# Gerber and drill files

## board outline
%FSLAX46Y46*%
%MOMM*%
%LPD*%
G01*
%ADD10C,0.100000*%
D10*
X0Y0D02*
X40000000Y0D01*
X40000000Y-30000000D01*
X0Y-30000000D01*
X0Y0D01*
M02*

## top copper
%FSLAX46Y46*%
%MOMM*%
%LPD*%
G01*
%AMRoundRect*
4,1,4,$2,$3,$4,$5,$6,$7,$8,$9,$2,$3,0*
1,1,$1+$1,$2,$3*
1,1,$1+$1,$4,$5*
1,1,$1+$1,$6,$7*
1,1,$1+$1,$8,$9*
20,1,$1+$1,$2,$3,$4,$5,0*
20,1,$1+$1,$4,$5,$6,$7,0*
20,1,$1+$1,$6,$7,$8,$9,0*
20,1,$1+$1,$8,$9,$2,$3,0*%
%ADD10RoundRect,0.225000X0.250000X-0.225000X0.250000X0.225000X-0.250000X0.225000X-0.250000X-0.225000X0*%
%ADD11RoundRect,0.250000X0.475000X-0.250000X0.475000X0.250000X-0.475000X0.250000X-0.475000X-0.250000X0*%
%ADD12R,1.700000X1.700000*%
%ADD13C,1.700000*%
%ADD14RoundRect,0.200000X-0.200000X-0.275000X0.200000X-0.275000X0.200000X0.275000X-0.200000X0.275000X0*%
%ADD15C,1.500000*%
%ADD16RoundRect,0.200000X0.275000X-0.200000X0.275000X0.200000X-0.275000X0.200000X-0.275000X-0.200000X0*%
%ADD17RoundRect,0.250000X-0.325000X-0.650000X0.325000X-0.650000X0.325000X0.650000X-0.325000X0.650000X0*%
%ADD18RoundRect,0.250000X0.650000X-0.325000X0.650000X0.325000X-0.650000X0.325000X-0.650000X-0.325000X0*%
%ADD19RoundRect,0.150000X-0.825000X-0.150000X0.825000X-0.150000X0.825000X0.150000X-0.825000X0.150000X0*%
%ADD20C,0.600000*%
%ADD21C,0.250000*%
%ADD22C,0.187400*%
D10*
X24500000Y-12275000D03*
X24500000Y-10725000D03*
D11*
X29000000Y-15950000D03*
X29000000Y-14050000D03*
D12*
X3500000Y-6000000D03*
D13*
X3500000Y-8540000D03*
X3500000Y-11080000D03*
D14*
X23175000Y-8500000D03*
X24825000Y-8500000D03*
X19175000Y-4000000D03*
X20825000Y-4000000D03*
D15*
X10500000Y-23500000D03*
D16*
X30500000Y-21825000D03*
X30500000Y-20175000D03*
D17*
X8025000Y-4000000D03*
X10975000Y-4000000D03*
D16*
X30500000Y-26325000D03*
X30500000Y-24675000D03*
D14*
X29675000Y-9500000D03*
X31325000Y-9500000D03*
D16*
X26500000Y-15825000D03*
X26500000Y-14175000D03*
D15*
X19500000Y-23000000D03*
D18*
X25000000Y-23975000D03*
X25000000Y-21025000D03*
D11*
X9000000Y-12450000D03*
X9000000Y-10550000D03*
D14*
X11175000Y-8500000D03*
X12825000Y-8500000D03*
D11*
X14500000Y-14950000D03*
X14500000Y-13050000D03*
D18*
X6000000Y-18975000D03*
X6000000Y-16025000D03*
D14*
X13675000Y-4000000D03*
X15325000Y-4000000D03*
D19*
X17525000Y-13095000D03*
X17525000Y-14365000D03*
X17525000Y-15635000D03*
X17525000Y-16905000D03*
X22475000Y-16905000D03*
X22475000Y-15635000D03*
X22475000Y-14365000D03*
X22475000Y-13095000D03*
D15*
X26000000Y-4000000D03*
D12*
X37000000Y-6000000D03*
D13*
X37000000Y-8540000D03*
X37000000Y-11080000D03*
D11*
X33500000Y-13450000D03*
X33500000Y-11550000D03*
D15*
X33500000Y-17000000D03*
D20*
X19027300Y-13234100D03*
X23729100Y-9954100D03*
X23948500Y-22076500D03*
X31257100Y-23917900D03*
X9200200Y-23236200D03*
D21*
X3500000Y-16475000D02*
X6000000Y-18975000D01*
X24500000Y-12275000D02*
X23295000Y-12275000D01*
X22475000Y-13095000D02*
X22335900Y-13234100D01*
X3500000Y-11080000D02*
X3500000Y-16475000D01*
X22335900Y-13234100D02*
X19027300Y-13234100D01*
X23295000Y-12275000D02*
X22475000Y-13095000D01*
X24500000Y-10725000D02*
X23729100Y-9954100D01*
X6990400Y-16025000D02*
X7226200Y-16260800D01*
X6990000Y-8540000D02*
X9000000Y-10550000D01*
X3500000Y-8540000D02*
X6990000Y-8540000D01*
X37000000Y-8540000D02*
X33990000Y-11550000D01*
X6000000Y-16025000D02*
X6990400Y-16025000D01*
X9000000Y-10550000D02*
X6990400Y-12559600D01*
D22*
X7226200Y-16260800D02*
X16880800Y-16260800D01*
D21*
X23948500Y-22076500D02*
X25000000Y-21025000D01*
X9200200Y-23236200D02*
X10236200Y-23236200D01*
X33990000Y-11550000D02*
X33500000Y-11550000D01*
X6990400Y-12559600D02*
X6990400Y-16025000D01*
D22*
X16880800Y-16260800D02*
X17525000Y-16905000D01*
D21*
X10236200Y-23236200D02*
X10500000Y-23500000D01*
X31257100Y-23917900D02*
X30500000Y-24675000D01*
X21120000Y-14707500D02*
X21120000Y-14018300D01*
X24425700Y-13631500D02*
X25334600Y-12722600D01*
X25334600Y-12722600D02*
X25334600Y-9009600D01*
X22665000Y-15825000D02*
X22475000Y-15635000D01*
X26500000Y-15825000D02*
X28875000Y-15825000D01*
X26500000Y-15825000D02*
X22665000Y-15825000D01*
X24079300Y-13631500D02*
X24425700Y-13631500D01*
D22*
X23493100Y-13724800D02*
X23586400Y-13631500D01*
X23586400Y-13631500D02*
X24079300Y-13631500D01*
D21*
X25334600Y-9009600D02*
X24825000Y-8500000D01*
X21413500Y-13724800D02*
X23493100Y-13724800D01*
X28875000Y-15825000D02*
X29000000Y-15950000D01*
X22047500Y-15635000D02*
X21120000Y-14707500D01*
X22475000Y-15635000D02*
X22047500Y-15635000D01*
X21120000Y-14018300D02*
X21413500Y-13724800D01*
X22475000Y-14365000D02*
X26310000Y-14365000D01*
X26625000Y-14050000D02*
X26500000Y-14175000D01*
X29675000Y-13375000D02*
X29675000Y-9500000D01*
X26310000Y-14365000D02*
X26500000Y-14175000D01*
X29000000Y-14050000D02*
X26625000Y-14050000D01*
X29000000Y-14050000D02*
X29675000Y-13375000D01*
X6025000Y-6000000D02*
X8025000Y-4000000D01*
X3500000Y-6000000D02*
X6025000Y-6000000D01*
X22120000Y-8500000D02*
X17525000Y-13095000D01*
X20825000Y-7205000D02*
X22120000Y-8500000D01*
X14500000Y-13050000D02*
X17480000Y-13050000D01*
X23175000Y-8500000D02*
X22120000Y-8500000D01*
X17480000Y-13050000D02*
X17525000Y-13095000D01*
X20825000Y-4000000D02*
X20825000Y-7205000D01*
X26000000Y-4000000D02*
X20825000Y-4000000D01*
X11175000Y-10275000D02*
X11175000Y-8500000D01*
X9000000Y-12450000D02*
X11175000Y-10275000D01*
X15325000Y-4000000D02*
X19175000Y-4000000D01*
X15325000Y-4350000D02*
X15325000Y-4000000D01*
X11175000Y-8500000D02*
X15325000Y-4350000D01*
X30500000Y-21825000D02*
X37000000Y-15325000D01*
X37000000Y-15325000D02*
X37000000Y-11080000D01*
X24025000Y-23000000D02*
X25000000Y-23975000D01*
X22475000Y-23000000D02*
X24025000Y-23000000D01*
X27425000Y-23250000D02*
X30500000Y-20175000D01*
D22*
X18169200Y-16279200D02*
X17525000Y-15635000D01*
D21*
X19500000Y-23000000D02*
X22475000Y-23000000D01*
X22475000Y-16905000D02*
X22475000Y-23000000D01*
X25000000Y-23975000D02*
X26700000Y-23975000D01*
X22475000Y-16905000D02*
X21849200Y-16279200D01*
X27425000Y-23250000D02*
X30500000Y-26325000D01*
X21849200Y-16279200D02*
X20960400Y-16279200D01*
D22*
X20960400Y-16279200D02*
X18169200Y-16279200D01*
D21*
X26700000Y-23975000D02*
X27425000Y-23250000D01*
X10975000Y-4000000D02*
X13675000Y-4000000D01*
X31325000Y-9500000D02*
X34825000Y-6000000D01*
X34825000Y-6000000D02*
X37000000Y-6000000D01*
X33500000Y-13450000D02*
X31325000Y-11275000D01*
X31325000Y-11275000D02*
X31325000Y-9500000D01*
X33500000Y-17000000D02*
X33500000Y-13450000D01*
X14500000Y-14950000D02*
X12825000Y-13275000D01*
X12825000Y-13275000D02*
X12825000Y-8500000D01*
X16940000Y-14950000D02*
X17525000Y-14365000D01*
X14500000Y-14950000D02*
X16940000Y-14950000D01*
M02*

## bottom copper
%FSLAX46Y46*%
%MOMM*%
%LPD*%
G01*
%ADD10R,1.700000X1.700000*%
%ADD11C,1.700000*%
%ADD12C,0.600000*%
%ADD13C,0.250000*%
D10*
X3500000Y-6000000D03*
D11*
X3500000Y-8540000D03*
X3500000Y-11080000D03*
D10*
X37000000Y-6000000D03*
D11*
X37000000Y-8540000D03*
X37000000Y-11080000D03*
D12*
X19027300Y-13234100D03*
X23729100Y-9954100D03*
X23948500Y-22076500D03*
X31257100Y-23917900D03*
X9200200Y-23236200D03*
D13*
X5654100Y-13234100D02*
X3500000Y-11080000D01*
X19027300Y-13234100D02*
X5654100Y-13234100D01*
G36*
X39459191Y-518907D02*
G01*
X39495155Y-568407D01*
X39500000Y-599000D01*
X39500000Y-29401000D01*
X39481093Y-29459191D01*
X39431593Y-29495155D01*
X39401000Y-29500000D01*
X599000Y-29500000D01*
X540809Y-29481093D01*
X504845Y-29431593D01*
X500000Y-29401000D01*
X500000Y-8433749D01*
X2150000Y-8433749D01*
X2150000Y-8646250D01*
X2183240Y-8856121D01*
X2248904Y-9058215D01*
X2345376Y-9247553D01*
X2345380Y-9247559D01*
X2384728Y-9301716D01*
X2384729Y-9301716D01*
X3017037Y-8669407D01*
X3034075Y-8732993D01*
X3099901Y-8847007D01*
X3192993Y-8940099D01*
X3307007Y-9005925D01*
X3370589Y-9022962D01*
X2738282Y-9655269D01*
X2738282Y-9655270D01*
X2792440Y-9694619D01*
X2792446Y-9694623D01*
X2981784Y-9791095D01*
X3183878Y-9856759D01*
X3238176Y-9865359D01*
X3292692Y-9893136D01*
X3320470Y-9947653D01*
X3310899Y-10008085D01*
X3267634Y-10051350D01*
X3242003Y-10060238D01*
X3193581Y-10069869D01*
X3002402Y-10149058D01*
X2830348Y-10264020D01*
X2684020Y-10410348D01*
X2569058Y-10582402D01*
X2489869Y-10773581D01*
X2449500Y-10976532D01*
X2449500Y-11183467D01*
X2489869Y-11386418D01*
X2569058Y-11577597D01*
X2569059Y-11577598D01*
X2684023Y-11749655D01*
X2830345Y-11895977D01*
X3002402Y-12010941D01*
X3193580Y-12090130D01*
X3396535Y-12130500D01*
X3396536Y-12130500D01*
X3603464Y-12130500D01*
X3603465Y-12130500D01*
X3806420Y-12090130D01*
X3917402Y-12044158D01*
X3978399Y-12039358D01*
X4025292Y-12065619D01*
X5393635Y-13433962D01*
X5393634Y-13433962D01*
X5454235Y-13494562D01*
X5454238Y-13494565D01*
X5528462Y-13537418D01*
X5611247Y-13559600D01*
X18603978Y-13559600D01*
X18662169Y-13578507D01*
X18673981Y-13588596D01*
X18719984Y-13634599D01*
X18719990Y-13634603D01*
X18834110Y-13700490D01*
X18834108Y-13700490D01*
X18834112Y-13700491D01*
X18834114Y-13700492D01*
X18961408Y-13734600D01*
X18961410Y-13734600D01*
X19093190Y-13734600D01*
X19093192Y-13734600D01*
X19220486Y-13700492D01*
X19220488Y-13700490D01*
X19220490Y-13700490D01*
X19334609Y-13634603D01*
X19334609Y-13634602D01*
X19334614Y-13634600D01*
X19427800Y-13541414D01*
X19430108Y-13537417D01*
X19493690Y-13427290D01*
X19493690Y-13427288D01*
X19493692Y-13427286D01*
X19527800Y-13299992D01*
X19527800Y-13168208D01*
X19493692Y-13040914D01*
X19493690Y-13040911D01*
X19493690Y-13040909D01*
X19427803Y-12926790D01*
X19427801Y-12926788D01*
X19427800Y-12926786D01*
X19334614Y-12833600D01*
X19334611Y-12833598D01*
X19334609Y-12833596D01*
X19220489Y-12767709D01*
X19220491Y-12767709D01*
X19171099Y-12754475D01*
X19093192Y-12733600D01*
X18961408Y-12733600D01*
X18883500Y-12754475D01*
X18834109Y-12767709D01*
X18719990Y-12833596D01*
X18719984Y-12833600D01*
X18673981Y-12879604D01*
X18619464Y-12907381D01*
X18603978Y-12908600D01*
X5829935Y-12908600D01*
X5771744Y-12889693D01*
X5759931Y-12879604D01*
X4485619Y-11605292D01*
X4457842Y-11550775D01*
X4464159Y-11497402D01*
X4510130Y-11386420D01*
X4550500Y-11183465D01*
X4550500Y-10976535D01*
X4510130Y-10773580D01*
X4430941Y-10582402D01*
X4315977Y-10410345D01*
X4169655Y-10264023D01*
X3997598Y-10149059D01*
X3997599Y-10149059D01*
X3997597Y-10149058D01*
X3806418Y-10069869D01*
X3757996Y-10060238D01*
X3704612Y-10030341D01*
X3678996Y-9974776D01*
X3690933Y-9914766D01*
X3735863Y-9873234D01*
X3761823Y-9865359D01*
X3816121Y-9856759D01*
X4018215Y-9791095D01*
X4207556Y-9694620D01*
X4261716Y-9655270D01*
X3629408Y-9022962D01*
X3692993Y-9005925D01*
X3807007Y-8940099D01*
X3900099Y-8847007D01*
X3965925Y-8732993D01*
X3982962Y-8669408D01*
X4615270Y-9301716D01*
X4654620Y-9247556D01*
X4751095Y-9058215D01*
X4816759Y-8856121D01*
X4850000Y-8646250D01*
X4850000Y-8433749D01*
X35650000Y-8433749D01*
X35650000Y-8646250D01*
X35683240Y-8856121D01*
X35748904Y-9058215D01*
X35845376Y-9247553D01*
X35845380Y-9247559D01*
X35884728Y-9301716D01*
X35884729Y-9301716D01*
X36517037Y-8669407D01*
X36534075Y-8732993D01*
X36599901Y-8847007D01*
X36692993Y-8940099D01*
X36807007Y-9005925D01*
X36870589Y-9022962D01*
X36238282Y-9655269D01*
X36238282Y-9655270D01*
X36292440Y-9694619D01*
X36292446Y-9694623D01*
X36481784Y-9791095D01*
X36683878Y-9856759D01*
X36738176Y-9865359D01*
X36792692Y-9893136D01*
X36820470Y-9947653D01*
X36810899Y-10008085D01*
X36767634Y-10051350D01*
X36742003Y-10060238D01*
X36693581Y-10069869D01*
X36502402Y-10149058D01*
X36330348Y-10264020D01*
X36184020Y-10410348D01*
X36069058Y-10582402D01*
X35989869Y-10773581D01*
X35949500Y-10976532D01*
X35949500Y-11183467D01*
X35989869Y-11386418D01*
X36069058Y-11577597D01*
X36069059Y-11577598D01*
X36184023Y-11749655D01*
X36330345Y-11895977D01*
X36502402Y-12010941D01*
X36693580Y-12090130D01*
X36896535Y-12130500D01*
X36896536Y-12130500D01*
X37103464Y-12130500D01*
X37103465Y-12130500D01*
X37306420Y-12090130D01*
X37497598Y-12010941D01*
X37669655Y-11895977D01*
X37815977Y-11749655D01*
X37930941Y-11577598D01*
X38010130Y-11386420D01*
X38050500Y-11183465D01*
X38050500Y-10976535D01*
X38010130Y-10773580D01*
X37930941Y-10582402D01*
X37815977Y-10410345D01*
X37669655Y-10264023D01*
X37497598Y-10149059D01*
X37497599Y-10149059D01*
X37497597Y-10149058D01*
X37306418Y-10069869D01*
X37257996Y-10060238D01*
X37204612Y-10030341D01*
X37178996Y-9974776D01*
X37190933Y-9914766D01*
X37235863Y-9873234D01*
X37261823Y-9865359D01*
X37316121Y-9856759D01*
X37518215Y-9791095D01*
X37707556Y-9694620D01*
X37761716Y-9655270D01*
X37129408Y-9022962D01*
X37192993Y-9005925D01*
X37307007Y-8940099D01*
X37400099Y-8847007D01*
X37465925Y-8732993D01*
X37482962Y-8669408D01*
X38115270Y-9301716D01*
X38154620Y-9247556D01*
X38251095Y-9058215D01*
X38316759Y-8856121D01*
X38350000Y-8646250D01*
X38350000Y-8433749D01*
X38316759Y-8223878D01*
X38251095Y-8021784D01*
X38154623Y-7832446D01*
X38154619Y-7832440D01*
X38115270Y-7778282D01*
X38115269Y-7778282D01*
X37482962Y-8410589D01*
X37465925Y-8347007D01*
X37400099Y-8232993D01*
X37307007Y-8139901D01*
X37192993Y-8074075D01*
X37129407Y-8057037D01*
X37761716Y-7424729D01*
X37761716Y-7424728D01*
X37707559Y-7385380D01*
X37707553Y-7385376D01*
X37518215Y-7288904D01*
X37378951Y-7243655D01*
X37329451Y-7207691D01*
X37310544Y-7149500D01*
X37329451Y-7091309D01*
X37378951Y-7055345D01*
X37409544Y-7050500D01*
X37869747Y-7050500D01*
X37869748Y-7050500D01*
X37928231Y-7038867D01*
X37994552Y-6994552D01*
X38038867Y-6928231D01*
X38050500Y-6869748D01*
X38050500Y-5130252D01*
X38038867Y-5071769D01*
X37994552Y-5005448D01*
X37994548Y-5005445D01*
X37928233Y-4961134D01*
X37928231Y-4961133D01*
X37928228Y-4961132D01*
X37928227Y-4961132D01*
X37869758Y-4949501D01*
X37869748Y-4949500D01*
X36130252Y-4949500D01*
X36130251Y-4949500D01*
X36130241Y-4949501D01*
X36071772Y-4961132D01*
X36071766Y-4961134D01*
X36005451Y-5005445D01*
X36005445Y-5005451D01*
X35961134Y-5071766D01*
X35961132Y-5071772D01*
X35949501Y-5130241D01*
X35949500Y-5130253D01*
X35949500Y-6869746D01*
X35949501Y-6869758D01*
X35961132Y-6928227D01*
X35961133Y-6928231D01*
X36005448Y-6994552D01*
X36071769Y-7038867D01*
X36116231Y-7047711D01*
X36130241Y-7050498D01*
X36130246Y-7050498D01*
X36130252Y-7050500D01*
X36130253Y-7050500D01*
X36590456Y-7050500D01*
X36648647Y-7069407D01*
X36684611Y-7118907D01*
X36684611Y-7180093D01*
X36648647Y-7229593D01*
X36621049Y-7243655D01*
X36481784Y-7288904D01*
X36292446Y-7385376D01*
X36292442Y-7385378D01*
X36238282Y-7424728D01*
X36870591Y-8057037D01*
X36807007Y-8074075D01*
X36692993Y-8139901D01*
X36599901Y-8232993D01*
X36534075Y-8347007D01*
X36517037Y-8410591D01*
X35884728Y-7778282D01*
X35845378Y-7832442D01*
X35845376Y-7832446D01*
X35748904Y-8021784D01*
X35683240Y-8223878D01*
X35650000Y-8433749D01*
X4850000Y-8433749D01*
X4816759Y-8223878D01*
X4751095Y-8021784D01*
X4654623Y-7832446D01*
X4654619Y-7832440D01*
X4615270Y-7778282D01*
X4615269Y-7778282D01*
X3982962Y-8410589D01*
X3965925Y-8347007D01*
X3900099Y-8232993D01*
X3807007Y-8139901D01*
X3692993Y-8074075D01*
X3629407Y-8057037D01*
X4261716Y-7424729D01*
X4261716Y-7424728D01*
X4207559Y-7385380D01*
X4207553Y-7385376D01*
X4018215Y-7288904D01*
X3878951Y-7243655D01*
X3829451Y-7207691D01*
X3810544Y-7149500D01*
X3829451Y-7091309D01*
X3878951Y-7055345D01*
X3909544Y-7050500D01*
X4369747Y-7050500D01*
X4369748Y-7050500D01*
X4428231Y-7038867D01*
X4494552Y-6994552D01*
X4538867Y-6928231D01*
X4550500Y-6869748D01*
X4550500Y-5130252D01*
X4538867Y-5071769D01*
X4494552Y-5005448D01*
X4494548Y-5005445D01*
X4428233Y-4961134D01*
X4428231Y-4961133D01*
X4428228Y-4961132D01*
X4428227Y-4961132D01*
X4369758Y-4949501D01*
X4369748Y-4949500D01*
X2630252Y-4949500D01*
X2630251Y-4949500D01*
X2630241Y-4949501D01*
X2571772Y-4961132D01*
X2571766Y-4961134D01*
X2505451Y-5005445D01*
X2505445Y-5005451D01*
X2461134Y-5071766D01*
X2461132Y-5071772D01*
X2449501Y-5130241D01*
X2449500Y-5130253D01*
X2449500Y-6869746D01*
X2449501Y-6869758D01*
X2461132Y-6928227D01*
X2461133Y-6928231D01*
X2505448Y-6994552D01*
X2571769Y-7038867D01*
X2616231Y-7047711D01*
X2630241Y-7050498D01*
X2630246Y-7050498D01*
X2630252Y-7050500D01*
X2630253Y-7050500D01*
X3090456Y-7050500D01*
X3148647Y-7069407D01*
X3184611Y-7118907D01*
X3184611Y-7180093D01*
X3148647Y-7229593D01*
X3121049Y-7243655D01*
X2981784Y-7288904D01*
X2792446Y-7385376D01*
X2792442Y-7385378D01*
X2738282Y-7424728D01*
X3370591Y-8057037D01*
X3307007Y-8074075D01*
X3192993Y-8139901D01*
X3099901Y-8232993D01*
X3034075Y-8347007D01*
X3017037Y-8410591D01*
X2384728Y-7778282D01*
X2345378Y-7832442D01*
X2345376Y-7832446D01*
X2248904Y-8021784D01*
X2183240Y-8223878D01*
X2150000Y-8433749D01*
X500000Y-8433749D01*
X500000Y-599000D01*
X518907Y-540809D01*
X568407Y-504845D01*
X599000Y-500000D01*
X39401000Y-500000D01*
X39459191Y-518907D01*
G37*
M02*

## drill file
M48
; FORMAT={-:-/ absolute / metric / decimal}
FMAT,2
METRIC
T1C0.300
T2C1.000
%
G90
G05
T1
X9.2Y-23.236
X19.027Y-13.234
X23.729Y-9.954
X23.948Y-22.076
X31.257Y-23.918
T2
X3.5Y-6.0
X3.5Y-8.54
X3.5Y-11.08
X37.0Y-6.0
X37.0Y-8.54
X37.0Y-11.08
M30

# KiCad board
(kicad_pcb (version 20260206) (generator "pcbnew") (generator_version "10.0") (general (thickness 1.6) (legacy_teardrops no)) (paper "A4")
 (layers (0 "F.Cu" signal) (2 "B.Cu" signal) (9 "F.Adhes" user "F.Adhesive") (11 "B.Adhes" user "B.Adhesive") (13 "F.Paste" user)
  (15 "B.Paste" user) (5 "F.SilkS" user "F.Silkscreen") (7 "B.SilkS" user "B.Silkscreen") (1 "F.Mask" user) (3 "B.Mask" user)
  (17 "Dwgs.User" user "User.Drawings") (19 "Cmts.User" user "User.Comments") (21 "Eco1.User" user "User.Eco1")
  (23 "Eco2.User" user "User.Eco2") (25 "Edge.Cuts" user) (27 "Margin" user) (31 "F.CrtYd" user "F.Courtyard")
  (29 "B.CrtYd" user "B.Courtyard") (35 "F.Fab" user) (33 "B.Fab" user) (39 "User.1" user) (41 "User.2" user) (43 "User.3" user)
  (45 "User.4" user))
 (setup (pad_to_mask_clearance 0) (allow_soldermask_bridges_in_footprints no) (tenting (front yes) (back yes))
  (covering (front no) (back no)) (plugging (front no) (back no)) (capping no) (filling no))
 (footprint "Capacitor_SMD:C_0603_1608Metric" (layer "F.Cu") (at 24.5 11.5 90)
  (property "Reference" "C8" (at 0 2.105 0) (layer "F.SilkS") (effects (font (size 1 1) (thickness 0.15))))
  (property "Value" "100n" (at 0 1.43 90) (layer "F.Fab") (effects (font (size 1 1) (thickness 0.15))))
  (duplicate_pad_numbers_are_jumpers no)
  (pad "1" smd roundrect (at -0.775 0 90) (size 0.9 0.95) (layers "F.Cu" "F.Mask" "F.Paste") (roundrect_rratio 0.25) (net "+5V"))
  (pad "2" smd roundrect (at 0.775 0 90) (size 0.9 0.95) (layers "F.Cu" "F.Mask" "F.Paste") (roundrect_rratio 0.25) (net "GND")))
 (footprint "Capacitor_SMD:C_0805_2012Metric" (layer "F.Cu") (at 29 15 90)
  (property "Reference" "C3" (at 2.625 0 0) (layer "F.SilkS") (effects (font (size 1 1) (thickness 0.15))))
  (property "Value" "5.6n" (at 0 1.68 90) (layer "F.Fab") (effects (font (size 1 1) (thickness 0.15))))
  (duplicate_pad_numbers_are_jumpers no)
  (pad "1" smd roundrect (at -0.95 0 90) (size 1 1.45) (layers "F.Cu" "F.Mask" "F.Paste") (roundrect_rratio 0.25) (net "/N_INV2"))
  (pad "2" smd roundrect (at 0.95 0 90) (size 1 1.45) (layers "F.Cu" "F.Mask" "F.Paste") (roundrect_rratio 0.25) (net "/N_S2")))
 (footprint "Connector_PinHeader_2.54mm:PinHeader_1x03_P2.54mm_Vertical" (layer "F.Cu") (at 3.5 6)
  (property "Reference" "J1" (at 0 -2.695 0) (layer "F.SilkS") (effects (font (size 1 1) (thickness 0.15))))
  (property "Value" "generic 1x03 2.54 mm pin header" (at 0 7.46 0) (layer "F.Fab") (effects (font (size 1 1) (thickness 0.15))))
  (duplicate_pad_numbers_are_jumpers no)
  (pad "1" thru_hole rect (at 0 0) (size 1.7 1.7) (drill 1) (layers "*.Cu" "*.Mask") (remove_unused_layers no) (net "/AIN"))
  (pad "2" thru_hole circle (at 0 2.54) (size 1.7 1.7) (drill 1) (layers "*.Cu" "*.Mask") (remove_unused_layers no) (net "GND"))
  (pad "3" thru_hole circle (at 0 5.08) (size 1.7 1.7) (drill 1) (layers "*.Cu" "*.Mask") (remove_unused_layers no) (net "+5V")))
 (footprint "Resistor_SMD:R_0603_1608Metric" (layer "F.Cu") (at 24 8.5)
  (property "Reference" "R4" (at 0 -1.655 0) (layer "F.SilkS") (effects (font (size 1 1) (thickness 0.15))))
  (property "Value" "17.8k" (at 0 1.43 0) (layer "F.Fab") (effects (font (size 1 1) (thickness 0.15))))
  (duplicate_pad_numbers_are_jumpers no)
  (pad "1" smd roundrect (at -0.825 0) (size 0.8 0.95) (layers "F.Cu" "F.Mask" "F.Paste") (roundrect_rratio 0.25) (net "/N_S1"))
  (pad "2" smd roundrect (at 0.825 0) (size 0.8 0.95) (layers "F.Cu" "F.Mask" "F.Paste") (roundrect_rratio 0.25) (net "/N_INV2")))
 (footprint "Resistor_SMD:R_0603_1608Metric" (layer "F.Cu") (at 20 4)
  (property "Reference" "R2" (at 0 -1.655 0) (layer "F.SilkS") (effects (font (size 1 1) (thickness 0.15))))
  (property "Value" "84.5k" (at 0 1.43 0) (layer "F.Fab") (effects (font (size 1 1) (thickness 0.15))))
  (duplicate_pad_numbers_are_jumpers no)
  (pad "1" smd roundrect (at -0.825 0) (size 0.8 0.95) (layers "F.Cu" "F.Mask" "F.Paste") (roundrect_rratio 0.25) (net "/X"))
  (pad "2" smd roundrect (at 0.825 0) (size 0.8 0.95) (layers "F.Cu" "F.Mask" "F.Paste") (roundrect_rratio 0.25) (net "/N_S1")))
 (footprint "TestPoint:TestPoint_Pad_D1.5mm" (layer "F.Cu") (at 10.5 23.5)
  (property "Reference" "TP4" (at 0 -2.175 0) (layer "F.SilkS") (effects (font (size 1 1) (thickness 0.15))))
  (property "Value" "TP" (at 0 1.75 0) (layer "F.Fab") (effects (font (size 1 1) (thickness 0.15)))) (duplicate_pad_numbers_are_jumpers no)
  (pad "1" smd circle (at 0 0) (size 1.5 1.5) (layers "F.Cu" "F.Mask") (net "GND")))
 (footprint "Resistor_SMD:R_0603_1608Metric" (layer "F.Cu") (at 30.5 21 90)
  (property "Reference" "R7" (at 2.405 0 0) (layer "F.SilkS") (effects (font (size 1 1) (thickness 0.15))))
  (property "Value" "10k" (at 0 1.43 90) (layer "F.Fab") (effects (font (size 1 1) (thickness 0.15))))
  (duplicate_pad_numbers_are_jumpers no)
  (pad "1" smd roundrect (at -0.825 0 90) (size 0.8 0.95) (layers "F.Cu" "F.Mask" "F.Paste") (roundrect_rratio 0.25) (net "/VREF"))
  (pad "2" smd roundrect (at 0.825 0 90) (size 0.8 0.95) (layers "F.Cu" "F.Mask" "F.Paste") (roundrect_rratio 0.25) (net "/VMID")))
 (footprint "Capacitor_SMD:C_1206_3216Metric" (layer "F.Cu") (at 9.5 4)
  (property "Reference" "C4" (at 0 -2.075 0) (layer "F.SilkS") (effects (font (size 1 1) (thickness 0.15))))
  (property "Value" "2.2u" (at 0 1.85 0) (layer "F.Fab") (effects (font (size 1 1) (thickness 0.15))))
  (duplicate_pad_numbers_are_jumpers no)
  (pad "1" smd roundrect (at -1.475 0) (size 1.15 1.8) (layers "F.Cu" "F.Mask" "F.Paste") (roundrect_rratio 0.217391) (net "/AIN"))
  (pad "2" smd roundrect (at 1.475 0) (size 1.15 1.8) (layers "F.Cu" "F.Mask" "F.Paste") (roundrect_rratio 0.217391) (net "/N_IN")))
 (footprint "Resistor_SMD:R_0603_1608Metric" (layer "F.Cu") (at 30.5 25.5 90)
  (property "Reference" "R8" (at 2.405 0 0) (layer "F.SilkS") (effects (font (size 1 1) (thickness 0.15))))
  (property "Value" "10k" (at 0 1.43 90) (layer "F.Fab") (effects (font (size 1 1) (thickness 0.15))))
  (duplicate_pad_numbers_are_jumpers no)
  (pad "1" smd roundrect (at -0.825 0 90) (size 0.8 0.95) (layers "F.Cu" "F.Mask" "F.Paste") (roundrect_rratio 0.25) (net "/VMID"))
  (pad "2" smd roundrect (at 0.825 0 90) (size 0.8 0.95) (layers "F.Cu" "F.Mask" "F.Paste") (roundrect_rratio 0.25) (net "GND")))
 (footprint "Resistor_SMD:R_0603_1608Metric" (layer "F.Cu") (at 30.5 9.5)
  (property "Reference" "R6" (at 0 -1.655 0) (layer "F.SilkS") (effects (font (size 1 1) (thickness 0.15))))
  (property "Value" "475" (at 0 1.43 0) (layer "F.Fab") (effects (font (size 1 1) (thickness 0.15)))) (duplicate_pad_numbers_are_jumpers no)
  (pad "1" smd roundrect (at -0.825 0) (size 0.8 0.95) (layers "F.Cu" "F.Mask" "F.Paste") (roundrect_rratio 0.25) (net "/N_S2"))
  (pad "2" smd roundrect (at 0.825 0) (size 0.8 0.95) (layers "F.Cu" "F.Mask" "F.Paste") (roundrect_rratio 0.25) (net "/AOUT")))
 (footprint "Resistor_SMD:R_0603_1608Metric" (layer "F.Cu") (at 26.5 15 90)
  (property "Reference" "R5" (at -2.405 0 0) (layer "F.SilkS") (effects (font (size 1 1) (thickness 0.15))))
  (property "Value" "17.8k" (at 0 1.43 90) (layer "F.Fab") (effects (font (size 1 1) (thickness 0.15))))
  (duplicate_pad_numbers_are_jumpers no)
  (pad "1" smd roundrect (at -0.825 0 90) (size 0.8 0.95) (layers "F.Cu" "F.Mask" "F.Paste") (roundrect_rratio 0.25) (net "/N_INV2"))
  (pad "2" smd roundrect (at 0.825 0 90) (size 0.8 0.95) (layers "F.Cu" "F.Mask" "F.Paste") (roundrect_rratio 0.25) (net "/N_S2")))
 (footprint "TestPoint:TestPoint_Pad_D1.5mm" (layer "F.Cu") (at 19.5 23)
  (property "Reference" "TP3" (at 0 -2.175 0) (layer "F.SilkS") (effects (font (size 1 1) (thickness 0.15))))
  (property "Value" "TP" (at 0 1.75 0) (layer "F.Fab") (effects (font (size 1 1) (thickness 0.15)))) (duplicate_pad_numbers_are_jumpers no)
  (pad "1" smd circle (at 0 0) (size 1.5 1.5) (layers "F.Cu" "F.Mask") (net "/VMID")))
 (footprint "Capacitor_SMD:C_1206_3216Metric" (layer "F.Cu") (at 25 22.5 90)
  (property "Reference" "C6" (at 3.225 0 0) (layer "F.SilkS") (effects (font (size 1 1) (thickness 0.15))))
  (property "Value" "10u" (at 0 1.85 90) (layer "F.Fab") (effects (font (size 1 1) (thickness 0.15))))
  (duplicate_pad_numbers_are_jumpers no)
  (pad "1" smd roundrect (at -1.475 0 90) (size 1.15 1.8) (layers "F.Cu" "F.Mask" "F.Paste") (roundrect_rratio 0.217391) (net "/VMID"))
  (pad "2" smd roundrect (at 1.475 0 90) (size 1.15 1.8) (layers "F.Cu" "F.Mask" "F.Paste") (roundrect_rratio 0.217391) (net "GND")))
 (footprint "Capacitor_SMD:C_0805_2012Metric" (layer "F.Cu") (at 9 11.5 90)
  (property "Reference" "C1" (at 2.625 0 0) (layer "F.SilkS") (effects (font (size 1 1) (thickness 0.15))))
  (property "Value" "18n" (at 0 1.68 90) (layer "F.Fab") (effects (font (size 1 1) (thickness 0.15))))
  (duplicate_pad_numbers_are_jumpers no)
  (pad "1" smd roundrect (at -0.95 0 90) (size 1 1.45) (layers "F.Cu" "F.Mask" "F.Paste") (roundrect_rratio 0.25) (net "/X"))
  (pad "2" smd roundrect (at 0.95 0 90) (size 1 1.45) (layers "F.Cu" "F.Mask" "F.Paste") (roundrect_rratio 0.25) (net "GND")))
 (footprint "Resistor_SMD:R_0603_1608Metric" (layer "F.Cu") (at 12 8.5)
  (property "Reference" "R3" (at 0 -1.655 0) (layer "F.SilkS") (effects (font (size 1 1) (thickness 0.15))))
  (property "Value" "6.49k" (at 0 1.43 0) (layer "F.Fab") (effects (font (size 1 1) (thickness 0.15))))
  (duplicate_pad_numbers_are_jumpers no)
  (pad "1" smd roundrect (at -0.825 0) (size 0.8 0.95) (layers "F.Cu" "F.Mask" "F.Paste") (roundrect_rratio 0.25) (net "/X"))
  (pad "2" smd roundrect (at 0.825 0) (size 0.8 0.95) (layers "F.Cu" "F.Mask" "F.Paste") (roundrect_rratio 0.25) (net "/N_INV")))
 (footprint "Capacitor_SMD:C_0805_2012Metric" (layer "F.Cu") (at 14.5 14 90)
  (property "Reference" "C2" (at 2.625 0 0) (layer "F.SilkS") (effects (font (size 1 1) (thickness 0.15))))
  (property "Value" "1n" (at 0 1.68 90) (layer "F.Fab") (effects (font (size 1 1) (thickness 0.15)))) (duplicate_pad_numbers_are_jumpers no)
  (pad "1" smd roundrect (at -0.95 0 90) (size 1 1.45) (layers "F.Cu" "F.Mask" "F.Paste") (roundrect_rratio 0.25) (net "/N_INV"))
  (pad "2" smd roundrect (at 0.95 0 90) (size 1 1.45) (layers "F.Cu" "F.Mask" "F.Paste") (roundrect_rratio 0.25) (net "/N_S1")))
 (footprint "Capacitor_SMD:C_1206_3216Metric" (layer "F.Cu") (at 6 17.5 90)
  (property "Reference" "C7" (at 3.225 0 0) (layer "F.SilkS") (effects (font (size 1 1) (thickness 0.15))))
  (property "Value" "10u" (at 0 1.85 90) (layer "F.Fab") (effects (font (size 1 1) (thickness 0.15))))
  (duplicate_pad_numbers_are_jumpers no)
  (pad "1" smd roundrect (at -1.475 0 90) (size 1.15 1.8) (layers "F.Cu" "F.Mask" "F.Paste") (roundrect_rratio 0.217391) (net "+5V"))
  (pad "2" smd roundrect (at 1.475 0 90) (size 1.15 1.8) (layers "F.Cu" "F.Mask" "F.Paste") (roundrect_rratio 0.217391) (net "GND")))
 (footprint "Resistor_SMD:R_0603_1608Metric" (layer "F.Cu") (at 14.5 4)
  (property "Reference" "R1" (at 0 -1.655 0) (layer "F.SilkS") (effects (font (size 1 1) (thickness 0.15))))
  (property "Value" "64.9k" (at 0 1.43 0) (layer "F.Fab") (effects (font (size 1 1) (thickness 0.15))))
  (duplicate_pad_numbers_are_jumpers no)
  (pad "1" smd roundrect (at -0.825 0) (size 0.8 0.95) (layers "F.Cu" "F.Mask" "F.Paste") (roundrect_rratio 0.25) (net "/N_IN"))
  (pad "2" smd roundrect (at 0.825 0) (size 0.8 0.95) (layers "F.Cu" "F.Mask" "F.Paste") (roundrect_rratio 0.25) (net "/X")))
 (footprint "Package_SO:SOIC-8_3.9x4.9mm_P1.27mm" (layer "F.Cu") (at 20 15)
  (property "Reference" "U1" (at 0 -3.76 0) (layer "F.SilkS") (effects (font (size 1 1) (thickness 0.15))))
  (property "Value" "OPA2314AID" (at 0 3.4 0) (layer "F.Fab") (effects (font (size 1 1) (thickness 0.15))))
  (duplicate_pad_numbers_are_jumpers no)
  (pad "1" smd roundrect (at -2.475 -1.905) (size 1.95 0.6) (layers "F.Cu" "F.Mask" "F.Paste") (roundrect_rratio 0.25) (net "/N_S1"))
  (pad "2" smd roundrect (at -2.475 -0.635) (size 1.95 0.6) (layers "F.Cu" "F.Mask" "F.Paste") (roundrect_rratio 0.25) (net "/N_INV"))
  (pad "3" smd roundrect (at -2.475 0.635) (size 1.95 0.6) (layers "F.Cu" "F.Mask" "F.Paste") (roundrect_rratio 0.25) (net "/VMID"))
  (pad "4" smd roundrect (at -2.475 1.905) (size 1.95 0.6) (layers "F.Cu" "F.Mask" "F.Paste") (roundrect_rratio 0.25) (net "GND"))
  (pad "5" smd roundrect (at 2.475 1.905) (size 1.95 0.6) (layers "F.Cu" "F.Mask" "F.Paste") (roundrect_rratio 0.25) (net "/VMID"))
  (pad "6" smd roundrect (at 2.475 0.635) (size 1.95 0.6) (layers "F.Cu" "F.Mask" "F.Paste") (roundrect_rratio 0.25) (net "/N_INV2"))
  (pad "7" smd roundrect (at 2.475 -0.635) (size 1.95 0.6) (layers "F.Cu" "F.Mask" "F.Paste") (roundrect_rratio 0.25) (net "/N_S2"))
  (pad "8" smd roundrect (at 2.475 -1.905) (size 1.95 0.6) (layers "F.Cu" "F.Mask" "F.Paste") (roundrect_rratio 0.25) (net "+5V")))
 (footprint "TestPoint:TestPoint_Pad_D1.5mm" (layer "F.Cu") (at 26 4)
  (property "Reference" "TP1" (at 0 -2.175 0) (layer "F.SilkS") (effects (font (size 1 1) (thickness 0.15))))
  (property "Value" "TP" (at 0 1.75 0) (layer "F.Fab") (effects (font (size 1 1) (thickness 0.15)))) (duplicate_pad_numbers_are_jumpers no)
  (pad "1" smd circle (at 0 0) (size 1.5 1.5) (layers "F.Cu" "F.Mask") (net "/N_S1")))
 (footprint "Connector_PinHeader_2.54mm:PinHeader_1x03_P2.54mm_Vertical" (layer "F.Cu") (at 37 6)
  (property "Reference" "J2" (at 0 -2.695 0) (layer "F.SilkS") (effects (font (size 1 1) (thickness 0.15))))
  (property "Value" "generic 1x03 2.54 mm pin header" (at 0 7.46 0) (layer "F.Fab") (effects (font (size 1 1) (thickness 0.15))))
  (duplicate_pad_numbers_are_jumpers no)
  (pad "1" thru_hole rect (at 0 0) (size 1.7 1.7) (drill 1) (layers "*.Cu" "*.Mask") (remove_unused_layers no) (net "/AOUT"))
  (pad "2" thru_hole circle (at 0 2.54) (size 1.7 1.7) (drill 1) (layers "*.Cu" "*.Mask") (remove_unused_layers no) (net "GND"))
  (pad "3" thru_hole circle (at 0 5.08) (size 1.7 1.7) (drill 1) (layers "*.Cu" "*.Mask") (remove_unused_layers no) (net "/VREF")))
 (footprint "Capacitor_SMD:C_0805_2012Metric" (layer "F.Cu") (at 33.5 12.5 90)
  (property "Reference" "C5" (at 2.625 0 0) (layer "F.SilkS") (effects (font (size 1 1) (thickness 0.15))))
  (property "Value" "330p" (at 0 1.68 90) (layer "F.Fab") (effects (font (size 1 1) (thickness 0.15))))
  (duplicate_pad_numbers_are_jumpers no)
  (pad "1" smd roundrect (at -0.95 0 90) (size 1 1.45) (layers "F.Cu" "F.Mask" "F.Paste") (roundrect_rratio 0.25) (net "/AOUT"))
  (pad "2" smd roundrect (at 0.95 0 90) (size 1 1.45) (layers "F.Cu" "F.Mask" "F.Paste") (roundrect_rratio 0.25) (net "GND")))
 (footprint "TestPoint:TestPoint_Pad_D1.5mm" (layer "F.Cu") (at 33.5 17)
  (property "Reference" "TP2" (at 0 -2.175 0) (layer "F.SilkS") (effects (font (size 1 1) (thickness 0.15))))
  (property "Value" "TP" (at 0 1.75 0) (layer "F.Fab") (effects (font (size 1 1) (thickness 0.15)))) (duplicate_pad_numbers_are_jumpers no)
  (pad "1" smd circle (at 0 0) (size 1.5 1.5) (layers "F.Cu" "F.Mask") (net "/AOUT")))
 (gr_rect (start 0 0) (end 40 30) (stroke (width 0.1) (type default)) (fill no) (layer "Edge.Cuts"))
 (segment (start 3.5 16.475) (end 6 18.975) (width 0.25) (layer "F.Cu") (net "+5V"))
 (segment (start 24.5 12.275) (end 23.295 12.275) (width 0.25) (layer "F.Cu") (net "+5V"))
 (segment (start 22.475 13.095) (end 22.3359 13.2341) (width 0.25) (layer "F.Cu") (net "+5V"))
 (segment (start 3.5 11.08) (end 3.5 16.475) (width 0.25) (layer "F.Cu") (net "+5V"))
 (segment (start 22.3359 13.2341) (end 19.0273 13.2341) (width 0.25) (layer "F.Cu") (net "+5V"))
 (segment (start 23.295 12.275) (end 22.475 13.095) (width 0.25) (layer "F.Cu") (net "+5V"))
 (via (at 19.0273 13.2341) (size 0.6) (drill 0.3) (layers "F.Cu" "B.Cu") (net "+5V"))
 (segment (start 5.6541 13.2341) (end 3.5 11.08) (width 0.25) (layer "B.Cu") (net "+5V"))
 (segment (start 19.0273 13.2341) (end 5.6541 13.2341) (width 0.25) (layer "B.Cu") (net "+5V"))
 (segment (start 24.5 10.725) (end 23.7291 9.9541) (width 0.25) (layer "F.Cu") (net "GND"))
 (segment (start 6.9904 16.025) (end 7.2262 16.2608) (width 0.25) (layer "F.Cu") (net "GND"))
 (segment (start 6.99 8.54) (end 9 10.55) (width 0.25) (layer "F.Cu") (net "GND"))
 (segment (start 3.5 8.54) (end 6.99 8.54) (width 0.25) (layer "F.Cu") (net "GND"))
 (segment (start 37 8.54) (end 33.99 11.55) (width 0.25) (layer "F.Cu") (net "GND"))
 (segment (start 6 16.025) (end 6.9904 16.025) (width 0.25) (layer "F.Cu") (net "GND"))
 (segment (start 9 10.55) (end 6.9904 12.5596) (width 0.25) (layer "F.Cu") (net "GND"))
 (segment (start 7.2262 16.2608) (end 16.8808 16.2608) (width 0.1874) (layer "F.Cu") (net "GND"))
 (segment (start 23.9485 22.0765) (end 25 21.025) (width 0.25) (layer "F.Cu") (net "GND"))
 (segment (start 9.2002 23.2362) (end 10.2362 23.2362) (width 0.25) (layer "F.Cu") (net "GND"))
 (segment (start 33.99 11.55) (end 33.5 11.55) (width 0.25) (layer "F.Cu") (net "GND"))
 (segment (start 6.9904 12.5596) (end 6.9904 16.025) (width 0.25) (layer "F.Cu") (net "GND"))
 (segment (start 16.8808 16.2608) (end 17.525 16.905) (width 0.1874) (layer "F.Cu") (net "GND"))
 (segment (start 10.2362 23.2362) (end 10.5 23.5) (width 0.25) (layer "F.Cu") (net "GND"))
 (segment (start 31.2571 23.9179) (end 30.5 24.675) (width 0.25) (layer "F.Cu") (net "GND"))
 (via (at 23.7291 9.9541) (size 0.6) (drill 0.3) (layers "F.Cu" "B.Cu") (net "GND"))
 (via (at 23.9485 22.0765) (size 0.6) (drill 0.3) (layers "F.Cu" "B.Cu") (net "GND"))
 (via (at 31.2571 23.9179) (size 0.6) (drill 0.3) (layers "F.Cu" "B.Cu") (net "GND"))
 (via (at 9.2002 23.2362) (size 0.6) (drill 0.3) (layers "F.Cu" "B.Cu") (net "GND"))
 (segment (start 21.12 14.7075) (end 21.12 14.0183) (width 0.25) (layer "F.Cu") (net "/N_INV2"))
 (segment (start 24.4257 13.6315) (end 25.3346 12.7226) (width 0.25) (layer "F.Cu") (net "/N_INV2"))
 (segment (start 25.3346 12.7226) (end 25.3346 9.0096) (width 0.25) (layer "F.Cu") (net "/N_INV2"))
 (segment (start 22.665 15.825) (end 22.475 15.635) (width 0.25) (layer "F.Cu") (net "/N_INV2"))
 (segment (start 26.5 15.825) (end 28.875 15.825) (width 0.25) (layer "F.Cu") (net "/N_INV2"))
 (segment (start 26.5 15.825) (end 22.665 15.825) (width 0.25) (layer "F.Cu") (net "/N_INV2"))
 (segment (start 24.0793 13.6315) (end 24.4257 13.6315) (width 0.25) (layer "F.Cu") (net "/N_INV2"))
 (segment (start 23.4931 13.7248) (end 23.5864 13.6315) (width 0.1874) (layer "F.Cu") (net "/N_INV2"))
 (segment (start 23.5864 13.6315) (end 24.0793 13.6315) (width 0.1874) (layer "F.Cu") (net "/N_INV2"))
 (segment (start 25.3346 9.0096) (end 24.825 8.5) (width 0.25) (layer "F.Cu") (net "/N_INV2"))
 (segment (start 21.4135 13.7248) (end 23.4931 13.7248) (width 0.25) (layer "F.Cu") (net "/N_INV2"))
 (segment (start 28.875 15.825) (end 29 15.95) (width 0.25) (layer "F.Cu") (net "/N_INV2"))
 (segment (start 22.0475 15.635) (end 21.12 14.7075) (width 0.25) (layer "F.Cu") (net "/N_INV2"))
 (segment (start 22.475 15.635) (end 22.0475 15.635) (width 0.25) (layer "F.Cu") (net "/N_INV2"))
 (segment (start 21.12 14.0183) (end 21.4135 13.7248) (width 0.25) (layer "F.Cu") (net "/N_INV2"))
 (segment (start 22.475 14.365) (end 26.31 14.365) (width 0.25) (layer "F.Cu") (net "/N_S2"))
 (segment (start 26.625 14.05) (end 26.5 14.175) (width 0.25) (layer "F.Cu") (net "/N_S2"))
 (segment (start 29.675 13.375) (end 29.675 9.5) (width 0.25) (layer "F.Cu") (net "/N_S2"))
 (segment (start 26.31 14.365) (end 26.5 14.175) (width 0.25) (layer "F.Cu") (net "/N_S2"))
 (segment (start 29 14.05) (end 26.625 14.05) (width 0.25) (layer "F.Cu") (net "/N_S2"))
 (segment (start 29 14.05) (end 29.675 13.375) (width 0.25) (layer "F.Cu") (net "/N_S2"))
 (segment (start 6.025 6) (end 8.025 4) (width 0.25) (layer "F.Cu") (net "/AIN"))
 (segment (start 3.5 6) (end 6.025 6) (width 0.25) (layer "F.Cu") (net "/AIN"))
 (segment (start 22.12 8.5) (end 17.525 13.095) (width 0.25) (layer "F.Cu") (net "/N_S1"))
 (segment (start 20.825 7.205) (end 22.12 8.5) (width 0.25) (layer "F.Cu") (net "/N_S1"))
 (segment (start 14.5 13.05) (end 17.48 13.05) (width 0.25) (layer "F.Cu") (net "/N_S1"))
 (segment (start 23.175 8.5) (end 22.12 8.5) (width 0.25) (layer "F.Cu") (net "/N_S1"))
 (segment (start 17.48 13.05) (end 17.525 13.095) (width 0.25) (layer "F.Cu") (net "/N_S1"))
 (segment (start 20.825 4) (end 20.825 7.205) (width 0.25) (layer "F.Cu") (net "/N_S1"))
 (segment (start 26 4) (end 20.825 4) (width 0.25) (layer "F.Cu") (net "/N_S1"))
 (segment (start 11.175 10.275) (end 11.175 8.5) (width 0.25) (layer "F.Cu") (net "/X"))
 (segment (start 9 12.45) (end 11.175 10.275) (width 0.25) (layer "F.Cu") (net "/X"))
 (segment (start 15.325 4) (end 19.175 4) (width 0.25) (layer "F.Cu") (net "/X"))
 (segment (start 15.325 4.35) (end 15.325 4) (width 0.25) (layer "F.Cu") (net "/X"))
 (segment (start 11.175 8.5) (end 15.325 4.35) (width 0.25) (layer "F.Cu") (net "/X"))
 (segment (start 30.5 21.825) (end 37 15.325) (width 0.25) (layer "F.Cu") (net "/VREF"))
 (segment (start 37 15.325) (end 37 11.08) (width 0.25) (layer "F.Cu") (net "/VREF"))
 (segment (start 24.025 23) (end 25 23.975) (width 0.25) (layer "F.Cu") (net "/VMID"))
 (segment (start 22.475 23) (end 24.025 23) (width 0.25) (layer "F.Cu") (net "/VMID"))
 (segment (start 27.425 23.25) (end 30.5 20.175) (width 0.25) (layer "F.Cu") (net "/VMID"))
 (segment (start 18.1692 16.2792) (end 17.525 15.635) (width 0.1874) (layer "F.Cu") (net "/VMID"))
 (segment (start 19.5 23) (end 22.475 23) (width 0.25) (layer "F.Cu") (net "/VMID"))
 (segment (start 22.475 16.905) (end 22.475 23) (width 0.25) (layer "F.Cu") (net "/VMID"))
 (segment (start 25 23.975) (end 26.7 23.975) (width 0.25) (layer "F.Cu") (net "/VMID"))
 (segment (start 22.475 16.905) (end 21.8492 16.2792) (width 0.25) (layer "F.Cu") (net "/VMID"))
 (segment (start 27.425 23.25) (end 30.5 26.325) (width 0.25) (layer "F.Cu") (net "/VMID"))
 (segment (start 21.8492 16.2792) (end 20.9604 16.2792) (width 0.25) (layer "F.Cu") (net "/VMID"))
 (segment (start 20.9604 16.2792) (end 18.1692 16.2792) (width 0.1874) (layer "F.Cu") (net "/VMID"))
 (segment (start 26.7 23.975) (end 27.425 23.25) (width 0.25) (layer "F.Cu") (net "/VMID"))
 (segment (start 10.975 4) (end 13.675 4) (width 0.25) (layer "F.Cu") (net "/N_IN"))
 (segment (start 31.325 9.5) (end 34.825 6) (width 0.25) (layer "F.Cu") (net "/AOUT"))
 (segment (start 34.825 6) (end 37 6) (width 0.25) (layer "F.Cu") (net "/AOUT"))
 (segment (start 33.5 13.45) (end 31.325 11.275) (width 0.25) (layer "F.Cu") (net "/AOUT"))
 (segment (start 31.325 11.275) (end 31.325 9.5) (width 0.25) (layer "F.Cu") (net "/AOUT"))
 (segment (start 33.5 17) (end 33.5 13.45) (width 0.25) (layer "F.Cu") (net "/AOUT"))
 (segment (start 14.5 14.95) (end 12.825 13.275) (width 0.25) (layer "F.Cu") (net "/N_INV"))
 (segment (start 12.825 13.275) (end 12.825 8.5) (width 0.25) (layer "F.Cu") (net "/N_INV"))
 (segment (start 16.94 14.95) (end 17.525 14.365) (width 0.25) (layer "F.Cu") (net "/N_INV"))
 (segment (start 14.5 14.95) (end 16.94 14.95) (width 0.25) (layer "F.Cu") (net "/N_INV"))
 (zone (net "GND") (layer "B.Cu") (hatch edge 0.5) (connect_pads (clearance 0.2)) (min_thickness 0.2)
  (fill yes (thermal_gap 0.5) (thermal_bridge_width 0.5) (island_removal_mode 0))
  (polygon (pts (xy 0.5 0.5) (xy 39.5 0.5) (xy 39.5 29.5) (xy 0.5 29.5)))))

